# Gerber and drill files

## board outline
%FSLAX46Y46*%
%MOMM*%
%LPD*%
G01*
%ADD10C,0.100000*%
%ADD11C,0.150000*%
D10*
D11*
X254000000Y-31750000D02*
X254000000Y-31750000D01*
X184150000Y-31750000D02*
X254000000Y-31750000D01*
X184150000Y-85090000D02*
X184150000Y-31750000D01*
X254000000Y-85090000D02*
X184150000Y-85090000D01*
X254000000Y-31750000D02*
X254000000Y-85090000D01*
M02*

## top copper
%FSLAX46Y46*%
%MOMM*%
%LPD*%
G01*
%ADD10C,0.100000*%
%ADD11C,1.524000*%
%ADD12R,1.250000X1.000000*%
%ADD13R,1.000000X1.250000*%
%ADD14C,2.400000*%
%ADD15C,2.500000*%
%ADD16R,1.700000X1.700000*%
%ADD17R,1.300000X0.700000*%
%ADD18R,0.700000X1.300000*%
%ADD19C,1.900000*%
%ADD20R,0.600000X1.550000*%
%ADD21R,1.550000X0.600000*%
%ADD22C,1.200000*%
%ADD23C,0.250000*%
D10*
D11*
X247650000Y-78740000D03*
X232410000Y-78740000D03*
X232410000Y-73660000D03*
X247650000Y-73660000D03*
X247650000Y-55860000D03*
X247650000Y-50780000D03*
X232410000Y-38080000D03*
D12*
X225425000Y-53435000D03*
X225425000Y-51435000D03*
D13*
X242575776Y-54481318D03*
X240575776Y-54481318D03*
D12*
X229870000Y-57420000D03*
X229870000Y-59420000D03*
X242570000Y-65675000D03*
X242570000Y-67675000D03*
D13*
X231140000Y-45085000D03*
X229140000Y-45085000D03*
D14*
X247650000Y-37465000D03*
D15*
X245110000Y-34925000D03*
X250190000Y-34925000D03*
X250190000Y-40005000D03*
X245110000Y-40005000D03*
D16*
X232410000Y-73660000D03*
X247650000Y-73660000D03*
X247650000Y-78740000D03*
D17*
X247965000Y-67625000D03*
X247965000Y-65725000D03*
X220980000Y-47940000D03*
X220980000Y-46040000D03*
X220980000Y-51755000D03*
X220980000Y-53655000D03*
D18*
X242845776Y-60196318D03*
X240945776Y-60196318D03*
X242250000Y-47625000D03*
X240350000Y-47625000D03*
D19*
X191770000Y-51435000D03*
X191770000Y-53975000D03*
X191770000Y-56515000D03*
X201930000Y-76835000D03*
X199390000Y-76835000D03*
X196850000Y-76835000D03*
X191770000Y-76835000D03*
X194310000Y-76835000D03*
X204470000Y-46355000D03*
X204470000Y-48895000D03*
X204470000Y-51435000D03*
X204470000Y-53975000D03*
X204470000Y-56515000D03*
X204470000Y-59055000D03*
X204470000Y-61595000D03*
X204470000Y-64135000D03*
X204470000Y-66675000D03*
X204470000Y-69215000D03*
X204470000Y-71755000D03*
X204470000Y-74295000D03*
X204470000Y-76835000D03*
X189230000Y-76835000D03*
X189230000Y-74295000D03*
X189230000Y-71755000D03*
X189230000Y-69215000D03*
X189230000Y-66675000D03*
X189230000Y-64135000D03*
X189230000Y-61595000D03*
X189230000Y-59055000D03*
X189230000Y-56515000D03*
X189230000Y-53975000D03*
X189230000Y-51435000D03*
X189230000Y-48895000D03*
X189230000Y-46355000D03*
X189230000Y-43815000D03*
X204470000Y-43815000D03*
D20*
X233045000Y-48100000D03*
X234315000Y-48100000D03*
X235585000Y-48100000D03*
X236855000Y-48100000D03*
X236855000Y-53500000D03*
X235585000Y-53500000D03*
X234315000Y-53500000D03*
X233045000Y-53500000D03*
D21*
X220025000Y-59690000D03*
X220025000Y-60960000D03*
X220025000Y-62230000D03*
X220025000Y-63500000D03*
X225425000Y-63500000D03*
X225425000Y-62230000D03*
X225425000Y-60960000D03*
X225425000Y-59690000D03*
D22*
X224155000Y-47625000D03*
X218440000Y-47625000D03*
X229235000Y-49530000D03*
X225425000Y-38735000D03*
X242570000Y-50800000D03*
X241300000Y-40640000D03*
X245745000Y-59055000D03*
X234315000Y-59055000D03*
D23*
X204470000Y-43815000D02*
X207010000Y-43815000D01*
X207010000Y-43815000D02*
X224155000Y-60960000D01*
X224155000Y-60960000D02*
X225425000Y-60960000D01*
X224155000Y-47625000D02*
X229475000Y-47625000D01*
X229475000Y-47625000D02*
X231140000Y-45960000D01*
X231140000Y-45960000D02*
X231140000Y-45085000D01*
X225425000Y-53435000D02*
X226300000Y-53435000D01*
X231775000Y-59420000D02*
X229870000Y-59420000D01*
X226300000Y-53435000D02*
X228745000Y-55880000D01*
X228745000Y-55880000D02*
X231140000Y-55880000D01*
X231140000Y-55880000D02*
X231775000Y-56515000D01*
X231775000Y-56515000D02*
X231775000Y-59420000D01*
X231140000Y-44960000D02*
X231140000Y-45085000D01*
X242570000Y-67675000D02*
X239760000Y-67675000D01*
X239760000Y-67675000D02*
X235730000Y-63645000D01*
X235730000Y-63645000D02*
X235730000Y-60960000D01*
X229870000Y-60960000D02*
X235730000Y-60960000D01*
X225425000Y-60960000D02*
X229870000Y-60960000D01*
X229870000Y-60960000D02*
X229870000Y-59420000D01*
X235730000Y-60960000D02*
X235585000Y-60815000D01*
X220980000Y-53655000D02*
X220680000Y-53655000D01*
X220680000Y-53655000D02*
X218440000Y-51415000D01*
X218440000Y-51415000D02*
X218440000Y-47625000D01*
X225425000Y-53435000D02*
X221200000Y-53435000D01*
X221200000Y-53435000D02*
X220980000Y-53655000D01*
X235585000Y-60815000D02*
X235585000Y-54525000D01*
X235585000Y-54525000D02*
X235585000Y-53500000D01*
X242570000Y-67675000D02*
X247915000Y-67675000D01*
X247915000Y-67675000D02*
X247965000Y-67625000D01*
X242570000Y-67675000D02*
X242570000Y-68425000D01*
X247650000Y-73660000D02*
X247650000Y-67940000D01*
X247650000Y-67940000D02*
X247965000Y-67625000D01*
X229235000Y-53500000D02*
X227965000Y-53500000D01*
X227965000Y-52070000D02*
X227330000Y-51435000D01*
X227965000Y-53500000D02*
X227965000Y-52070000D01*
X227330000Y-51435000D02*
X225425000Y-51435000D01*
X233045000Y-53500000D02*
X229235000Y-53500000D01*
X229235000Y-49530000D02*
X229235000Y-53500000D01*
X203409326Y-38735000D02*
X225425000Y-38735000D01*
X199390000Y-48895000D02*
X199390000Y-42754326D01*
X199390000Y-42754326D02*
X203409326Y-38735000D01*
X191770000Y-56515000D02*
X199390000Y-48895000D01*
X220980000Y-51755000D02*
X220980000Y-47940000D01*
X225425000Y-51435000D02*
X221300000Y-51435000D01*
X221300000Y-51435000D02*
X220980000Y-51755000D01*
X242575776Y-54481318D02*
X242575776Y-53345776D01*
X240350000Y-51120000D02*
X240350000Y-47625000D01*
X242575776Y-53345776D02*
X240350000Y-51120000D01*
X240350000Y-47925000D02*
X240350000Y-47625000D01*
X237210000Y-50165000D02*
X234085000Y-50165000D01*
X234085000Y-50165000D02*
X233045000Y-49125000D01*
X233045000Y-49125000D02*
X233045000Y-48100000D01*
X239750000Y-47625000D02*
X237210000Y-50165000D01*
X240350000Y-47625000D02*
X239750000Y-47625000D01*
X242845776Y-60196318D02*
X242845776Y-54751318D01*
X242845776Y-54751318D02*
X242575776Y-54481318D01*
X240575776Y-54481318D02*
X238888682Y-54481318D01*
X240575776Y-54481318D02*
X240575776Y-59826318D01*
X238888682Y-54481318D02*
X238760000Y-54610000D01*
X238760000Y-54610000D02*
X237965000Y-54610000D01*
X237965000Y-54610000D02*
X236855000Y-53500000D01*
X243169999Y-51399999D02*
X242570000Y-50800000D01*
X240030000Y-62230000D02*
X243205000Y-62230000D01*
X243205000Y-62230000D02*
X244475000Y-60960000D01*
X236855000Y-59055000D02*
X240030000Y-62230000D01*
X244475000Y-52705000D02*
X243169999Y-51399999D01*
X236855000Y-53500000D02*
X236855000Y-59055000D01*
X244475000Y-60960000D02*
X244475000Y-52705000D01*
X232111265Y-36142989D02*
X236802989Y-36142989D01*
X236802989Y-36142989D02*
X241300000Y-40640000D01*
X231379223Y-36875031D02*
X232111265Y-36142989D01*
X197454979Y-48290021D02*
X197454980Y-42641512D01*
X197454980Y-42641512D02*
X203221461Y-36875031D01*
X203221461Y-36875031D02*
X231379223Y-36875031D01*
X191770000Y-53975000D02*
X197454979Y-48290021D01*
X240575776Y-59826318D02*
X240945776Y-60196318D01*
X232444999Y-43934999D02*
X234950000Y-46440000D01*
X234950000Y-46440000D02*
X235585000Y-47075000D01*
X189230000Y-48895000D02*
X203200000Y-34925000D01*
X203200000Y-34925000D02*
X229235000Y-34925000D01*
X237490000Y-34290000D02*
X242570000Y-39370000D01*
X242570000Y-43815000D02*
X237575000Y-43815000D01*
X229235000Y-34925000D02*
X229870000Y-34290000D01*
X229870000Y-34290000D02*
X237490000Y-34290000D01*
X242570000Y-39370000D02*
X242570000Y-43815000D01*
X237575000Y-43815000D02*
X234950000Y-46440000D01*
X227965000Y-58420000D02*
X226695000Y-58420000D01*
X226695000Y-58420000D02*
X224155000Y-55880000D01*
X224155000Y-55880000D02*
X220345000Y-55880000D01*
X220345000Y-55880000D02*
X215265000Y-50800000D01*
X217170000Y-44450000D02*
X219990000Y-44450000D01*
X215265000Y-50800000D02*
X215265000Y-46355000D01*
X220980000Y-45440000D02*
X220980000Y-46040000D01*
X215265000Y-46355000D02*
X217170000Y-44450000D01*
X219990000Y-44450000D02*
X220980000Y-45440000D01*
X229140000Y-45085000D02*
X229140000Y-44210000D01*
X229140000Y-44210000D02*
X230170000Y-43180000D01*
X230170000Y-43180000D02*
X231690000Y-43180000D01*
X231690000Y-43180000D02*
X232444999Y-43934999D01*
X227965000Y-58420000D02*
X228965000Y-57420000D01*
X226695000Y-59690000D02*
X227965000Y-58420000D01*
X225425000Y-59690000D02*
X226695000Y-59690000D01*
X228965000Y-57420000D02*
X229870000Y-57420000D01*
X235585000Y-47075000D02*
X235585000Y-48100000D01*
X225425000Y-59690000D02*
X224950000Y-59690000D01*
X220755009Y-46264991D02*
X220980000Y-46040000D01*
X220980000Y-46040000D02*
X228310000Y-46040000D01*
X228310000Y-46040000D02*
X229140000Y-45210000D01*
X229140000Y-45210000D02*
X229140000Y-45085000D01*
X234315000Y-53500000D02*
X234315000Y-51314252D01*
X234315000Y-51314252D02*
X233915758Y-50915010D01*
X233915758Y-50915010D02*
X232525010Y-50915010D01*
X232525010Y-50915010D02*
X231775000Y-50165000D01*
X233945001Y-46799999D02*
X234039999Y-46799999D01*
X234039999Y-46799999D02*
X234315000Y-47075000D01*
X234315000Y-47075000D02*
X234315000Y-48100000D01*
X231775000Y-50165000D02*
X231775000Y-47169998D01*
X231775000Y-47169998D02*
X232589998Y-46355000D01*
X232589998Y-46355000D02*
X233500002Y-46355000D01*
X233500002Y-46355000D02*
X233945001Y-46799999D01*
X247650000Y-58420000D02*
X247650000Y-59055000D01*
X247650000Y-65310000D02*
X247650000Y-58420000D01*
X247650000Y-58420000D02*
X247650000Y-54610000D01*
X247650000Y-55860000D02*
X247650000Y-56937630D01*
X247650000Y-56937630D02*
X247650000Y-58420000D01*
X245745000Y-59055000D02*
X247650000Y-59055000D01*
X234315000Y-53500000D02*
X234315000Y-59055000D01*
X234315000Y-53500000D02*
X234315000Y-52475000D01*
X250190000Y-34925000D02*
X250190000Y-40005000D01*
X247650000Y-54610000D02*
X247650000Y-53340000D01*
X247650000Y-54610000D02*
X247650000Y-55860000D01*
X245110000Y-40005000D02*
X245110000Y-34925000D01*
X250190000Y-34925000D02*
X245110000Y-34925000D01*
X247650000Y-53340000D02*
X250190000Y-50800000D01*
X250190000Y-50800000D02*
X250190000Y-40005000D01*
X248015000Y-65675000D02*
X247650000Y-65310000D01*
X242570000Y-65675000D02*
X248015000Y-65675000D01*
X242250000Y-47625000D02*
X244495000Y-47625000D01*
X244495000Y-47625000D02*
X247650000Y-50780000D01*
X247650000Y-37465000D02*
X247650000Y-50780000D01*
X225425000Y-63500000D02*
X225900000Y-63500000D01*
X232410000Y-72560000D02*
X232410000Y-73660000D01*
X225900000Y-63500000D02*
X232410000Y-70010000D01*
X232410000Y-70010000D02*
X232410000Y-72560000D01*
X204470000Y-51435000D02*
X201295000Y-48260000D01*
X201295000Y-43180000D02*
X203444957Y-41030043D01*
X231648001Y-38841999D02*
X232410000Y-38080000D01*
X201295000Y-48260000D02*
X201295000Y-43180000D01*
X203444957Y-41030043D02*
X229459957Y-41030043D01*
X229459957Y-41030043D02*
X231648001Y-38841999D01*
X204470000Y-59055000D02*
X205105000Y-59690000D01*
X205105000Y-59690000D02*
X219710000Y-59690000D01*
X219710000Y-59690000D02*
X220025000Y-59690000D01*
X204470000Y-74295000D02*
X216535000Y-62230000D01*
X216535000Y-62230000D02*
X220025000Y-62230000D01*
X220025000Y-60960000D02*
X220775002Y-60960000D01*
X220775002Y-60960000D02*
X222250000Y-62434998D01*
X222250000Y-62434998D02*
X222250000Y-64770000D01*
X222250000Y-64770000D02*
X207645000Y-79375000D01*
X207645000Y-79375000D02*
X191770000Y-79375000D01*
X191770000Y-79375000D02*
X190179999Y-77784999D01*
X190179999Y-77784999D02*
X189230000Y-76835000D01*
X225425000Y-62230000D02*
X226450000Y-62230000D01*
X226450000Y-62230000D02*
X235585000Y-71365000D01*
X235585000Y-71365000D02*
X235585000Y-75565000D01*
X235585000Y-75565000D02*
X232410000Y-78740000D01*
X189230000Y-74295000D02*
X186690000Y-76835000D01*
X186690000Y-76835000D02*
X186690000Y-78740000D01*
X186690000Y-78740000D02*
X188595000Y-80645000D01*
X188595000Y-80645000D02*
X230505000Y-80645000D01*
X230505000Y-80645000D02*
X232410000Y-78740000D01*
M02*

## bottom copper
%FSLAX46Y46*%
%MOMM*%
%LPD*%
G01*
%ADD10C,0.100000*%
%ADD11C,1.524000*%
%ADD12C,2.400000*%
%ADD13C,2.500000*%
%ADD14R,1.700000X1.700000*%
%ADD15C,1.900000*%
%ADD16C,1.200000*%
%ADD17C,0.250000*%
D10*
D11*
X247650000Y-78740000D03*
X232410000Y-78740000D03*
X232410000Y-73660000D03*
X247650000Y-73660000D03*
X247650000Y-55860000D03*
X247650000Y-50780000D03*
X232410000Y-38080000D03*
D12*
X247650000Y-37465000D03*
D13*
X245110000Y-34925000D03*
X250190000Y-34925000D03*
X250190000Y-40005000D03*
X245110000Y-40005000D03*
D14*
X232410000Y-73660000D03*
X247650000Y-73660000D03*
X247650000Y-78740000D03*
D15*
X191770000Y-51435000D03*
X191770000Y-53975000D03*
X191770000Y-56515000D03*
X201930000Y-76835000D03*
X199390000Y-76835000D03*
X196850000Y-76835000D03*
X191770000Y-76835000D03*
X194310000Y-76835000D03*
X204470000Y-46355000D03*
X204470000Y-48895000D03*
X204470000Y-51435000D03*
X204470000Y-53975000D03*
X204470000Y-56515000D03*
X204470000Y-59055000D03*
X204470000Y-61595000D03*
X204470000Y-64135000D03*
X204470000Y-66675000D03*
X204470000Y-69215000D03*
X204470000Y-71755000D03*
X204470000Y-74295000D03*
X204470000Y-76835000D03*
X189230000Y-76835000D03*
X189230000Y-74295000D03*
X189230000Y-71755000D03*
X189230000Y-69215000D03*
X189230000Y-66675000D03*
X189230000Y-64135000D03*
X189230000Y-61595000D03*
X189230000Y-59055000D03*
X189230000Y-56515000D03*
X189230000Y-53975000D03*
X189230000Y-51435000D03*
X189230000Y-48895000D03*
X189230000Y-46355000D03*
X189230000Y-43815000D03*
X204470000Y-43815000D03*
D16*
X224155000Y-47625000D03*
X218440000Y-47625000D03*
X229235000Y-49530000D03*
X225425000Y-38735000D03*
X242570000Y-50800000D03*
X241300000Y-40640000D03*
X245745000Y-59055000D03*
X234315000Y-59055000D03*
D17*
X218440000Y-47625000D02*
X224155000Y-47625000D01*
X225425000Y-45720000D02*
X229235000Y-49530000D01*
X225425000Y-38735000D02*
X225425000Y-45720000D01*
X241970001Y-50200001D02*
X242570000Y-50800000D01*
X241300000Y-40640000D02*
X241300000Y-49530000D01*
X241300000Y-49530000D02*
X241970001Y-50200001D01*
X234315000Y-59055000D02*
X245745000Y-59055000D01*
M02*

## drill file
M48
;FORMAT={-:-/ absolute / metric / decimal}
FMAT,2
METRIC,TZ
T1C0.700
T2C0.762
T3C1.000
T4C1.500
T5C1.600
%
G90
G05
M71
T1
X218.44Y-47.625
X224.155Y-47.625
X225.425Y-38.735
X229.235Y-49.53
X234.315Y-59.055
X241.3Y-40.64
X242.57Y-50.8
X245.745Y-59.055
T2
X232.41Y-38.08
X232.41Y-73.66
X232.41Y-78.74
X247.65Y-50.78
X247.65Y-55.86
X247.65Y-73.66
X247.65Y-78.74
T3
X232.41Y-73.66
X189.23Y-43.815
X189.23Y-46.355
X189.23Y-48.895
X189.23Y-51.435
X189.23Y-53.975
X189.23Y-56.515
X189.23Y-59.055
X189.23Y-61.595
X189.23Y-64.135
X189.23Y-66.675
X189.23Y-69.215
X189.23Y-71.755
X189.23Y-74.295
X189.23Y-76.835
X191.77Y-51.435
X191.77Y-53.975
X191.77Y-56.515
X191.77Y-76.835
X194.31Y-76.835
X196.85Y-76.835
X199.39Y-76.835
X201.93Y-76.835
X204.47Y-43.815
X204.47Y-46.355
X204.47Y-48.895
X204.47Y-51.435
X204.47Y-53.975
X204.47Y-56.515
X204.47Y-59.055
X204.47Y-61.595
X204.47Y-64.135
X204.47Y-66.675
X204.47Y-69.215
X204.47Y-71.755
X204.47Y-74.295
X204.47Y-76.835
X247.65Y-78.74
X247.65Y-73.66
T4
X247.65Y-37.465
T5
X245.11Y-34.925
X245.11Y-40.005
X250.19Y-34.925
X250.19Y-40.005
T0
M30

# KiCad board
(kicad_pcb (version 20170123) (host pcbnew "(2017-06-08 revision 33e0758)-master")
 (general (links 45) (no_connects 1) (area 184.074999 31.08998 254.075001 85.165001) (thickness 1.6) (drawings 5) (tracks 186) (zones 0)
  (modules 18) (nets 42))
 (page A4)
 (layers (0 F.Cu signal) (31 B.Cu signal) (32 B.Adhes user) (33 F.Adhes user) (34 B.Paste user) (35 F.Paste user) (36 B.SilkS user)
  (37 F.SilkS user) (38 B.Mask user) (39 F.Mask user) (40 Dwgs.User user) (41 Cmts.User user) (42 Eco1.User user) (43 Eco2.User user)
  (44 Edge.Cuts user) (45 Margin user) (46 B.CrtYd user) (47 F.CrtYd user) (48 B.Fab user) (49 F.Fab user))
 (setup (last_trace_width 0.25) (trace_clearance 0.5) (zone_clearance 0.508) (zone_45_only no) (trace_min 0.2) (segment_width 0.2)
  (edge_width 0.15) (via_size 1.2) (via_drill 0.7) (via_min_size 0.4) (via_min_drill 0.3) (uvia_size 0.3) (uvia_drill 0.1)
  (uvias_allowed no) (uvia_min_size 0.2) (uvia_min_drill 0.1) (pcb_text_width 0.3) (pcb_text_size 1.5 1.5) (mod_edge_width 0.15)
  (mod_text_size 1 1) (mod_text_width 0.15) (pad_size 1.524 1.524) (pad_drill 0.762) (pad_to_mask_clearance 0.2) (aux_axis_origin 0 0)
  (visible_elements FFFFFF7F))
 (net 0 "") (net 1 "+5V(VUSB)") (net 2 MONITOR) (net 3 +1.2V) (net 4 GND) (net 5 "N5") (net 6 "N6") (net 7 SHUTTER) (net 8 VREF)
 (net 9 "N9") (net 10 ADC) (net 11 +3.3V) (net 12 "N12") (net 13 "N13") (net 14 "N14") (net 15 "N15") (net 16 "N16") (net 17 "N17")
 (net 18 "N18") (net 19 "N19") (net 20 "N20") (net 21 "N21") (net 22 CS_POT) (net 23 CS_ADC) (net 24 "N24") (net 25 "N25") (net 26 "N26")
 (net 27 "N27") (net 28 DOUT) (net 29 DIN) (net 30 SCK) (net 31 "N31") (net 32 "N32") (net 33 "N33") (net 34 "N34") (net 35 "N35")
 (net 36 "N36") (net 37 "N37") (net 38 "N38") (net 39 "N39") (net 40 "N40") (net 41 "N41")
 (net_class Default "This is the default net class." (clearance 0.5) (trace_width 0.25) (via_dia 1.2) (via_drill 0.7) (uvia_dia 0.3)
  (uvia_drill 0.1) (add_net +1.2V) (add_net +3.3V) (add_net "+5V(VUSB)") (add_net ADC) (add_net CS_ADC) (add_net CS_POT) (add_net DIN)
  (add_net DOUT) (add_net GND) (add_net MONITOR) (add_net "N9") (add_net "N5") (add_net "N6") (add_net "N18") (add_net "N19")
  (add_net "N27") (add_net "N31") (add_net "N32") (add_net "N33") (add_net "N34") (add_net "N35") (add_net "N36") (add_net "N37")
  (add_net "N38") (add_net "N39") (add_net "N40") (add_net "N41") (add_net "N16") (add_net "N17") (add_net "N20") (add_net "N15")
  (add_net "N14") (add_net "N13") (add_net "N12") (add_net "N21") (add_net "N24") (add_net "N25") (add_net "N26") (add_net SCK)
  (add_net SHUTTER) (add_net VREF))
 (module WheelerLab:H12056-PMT (layer B.Cu) (at 232.41 38.08 270)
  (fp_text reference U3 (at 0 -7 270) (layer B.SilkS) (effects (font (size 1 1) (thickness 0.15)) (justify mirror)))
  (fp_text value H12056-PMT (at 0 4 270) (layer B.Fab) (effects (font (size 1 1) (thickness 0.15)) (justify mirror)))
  (pad 4 thru_hole circle (at 40.66 -15.24 270) (size 1.524 1.524) (drill 0.762) (layers *.Cu *.Mask) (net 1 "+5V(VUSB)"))
  (pad 3 thru_hole circle (at 40.66 0 270) (size 1.524 1.524) (drill 0.762) (layers *.Cu *.Mask) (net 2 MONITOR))
  (pad 2 thru_hole circle (at 35.58 0 270) (size 1.524 1.524) (drill 0.762) (layers *.Cu *.Mask) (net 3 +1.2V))
  (pad 5 thru_hole circle (at 35.58 -15.24 270) (size 1.524 1.524) (drill 0.762) (layers *.Cu *.Mask) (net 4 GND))
  (pad 6 thru_hole circle (at 17.78 -15.24 270) (size 1.524 1.524) (drill 0.762) (layers *.Cu *.Mask) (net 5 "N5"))
  (pad 7 thru_hole circle (at 12.7 -15.24 270) (size 1.524 1.524) (drill 0.762) (layers *.Cu *.Mask) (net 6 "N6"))
  (pad 1 thru_hole circle (at 0 0 270) (size 1.524 1.524) (drill 0.762) (layers *.Cu *.Mask) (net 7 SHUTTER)))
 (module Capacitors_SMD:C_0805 (layer F.Cu) (at 225.425 52.435 90)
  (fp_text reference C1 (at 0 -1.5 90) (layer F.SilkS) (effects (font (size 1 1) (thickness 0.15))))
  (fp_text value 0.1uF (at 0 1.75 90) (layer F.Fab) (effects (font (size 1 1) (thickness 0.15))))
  (pad 1 smd rect (at -1 0 90) (size 1 1.25) (layers F.Cu F.Paste F.Mask) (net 4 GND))
  (pad 2 smd rect (at 1 0 90) (size 1 1.25) (layers F.Cu F.Paste F.Mask) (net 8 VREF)))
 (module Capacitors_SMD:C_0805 (layer F.Cu) (at 241.575776 54.481318)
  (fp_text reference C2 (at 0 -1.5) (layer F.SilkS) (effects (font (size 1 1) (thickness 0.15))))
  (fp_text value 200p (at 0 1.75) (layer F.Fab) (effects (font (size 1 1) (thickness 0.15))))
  (pad 2 smd rect (at 1 0) (size 1 1.25) (layers F.Cu F.Paste F.Mask) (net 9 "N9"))
  (pad 1 smd rect (at -1 0) (size 1 1.25) (layers F.Cu F.Paste F.Mask) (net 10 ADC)))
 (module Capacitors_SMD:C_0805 (layer F.Cu) (at 229.87 58.42 90)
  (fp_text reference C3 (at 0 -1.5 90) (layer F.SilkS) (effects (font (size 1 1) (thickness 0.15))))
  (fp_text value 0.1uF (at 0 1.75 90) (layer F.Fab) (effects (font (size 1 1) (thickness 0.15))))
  (pad 2 smd rect (at 1 0 90) (size 1 1.25) (layers F.Cu F.Paste F.Mask) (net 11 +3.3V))
  (pad 1 smd rect (at -1 0 90) (size 1 1.25) (layers F.Cu F.Paste F.Mask) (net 4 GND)))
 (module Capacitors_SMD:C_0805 (layer F.Cu) (at 242.57 66.675 270)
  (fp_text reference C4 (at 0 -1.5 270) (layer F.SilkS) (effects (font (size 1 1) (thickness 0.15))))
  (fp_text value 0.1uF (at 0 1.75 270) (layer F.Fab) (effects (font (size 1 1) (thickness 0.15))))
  (pad 1 smd rect (at -1 0 270) (size 1 1.25) (layers F.Cu F.Paste F.Mask) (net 5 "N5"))
  (pad 2 smd rect (at 1 0 270) (size 1 1.25) (layers F.Cu F.Paste F.Mask) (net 4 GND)))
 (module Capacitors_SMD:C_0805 (layer F.Cu) (at 230.14 45.085)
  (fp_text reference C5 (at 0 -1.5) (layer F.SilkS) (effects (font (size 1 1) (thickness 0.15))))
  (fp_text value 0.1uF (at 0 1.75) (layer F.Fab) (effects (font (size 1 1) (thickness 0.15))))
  (pad 2 smd rect (at 1 0) (size 1 1.25) (layers F.Cu F.Paste F.Mask) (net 4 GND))
  (pad 1 smd rect (at -1 0) (size 1 1.25) (layers F.Cu F.Paste F.Mask) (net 11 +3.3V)))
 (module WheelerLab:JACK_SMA (layer F.Cu) (at 247.65 37.465)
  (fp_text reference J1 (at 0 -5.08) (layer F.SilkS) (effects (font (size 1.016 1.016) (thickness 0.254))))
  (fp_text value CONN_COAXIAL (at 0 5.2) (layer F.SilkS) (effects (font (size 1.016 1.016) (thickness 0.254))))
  (pad 1 thru_hole circle (at 0 0) (size 2.4 2.4) (drill 1.5) (layers *.Cu *.Mask F.SilkS) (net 6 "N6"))
  (pad 2 thru_hole circle (at -2.54 -2.54) (size 2.5 2.5) (drill 1.6) (layers *.Cu *.Mask F.SilkS) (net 5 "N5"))
  (pad 2 thru_hole circle (at 2.54 -2.54) (size 2.5 2.5) (drill 1.6) (layers *.Cu *.Mask F.SilkS) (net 5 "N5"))
  (pad 2 thru_hole circle (at 2.54 2.54) (size 2.5 2.5) (drill 1.6) (layers *.Cu *.Mask F.SilkS) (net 5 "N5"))
  (pad 2 thru_hole circle (at -2.54 2.54) (size 2.5 2.5) (drill 1.6) (layers *.Cu *.Mask F.SilkS) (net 5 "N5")))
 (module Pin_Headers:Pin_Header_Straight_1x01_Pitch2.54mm (layer F.Cu) (at 232.41 73.66)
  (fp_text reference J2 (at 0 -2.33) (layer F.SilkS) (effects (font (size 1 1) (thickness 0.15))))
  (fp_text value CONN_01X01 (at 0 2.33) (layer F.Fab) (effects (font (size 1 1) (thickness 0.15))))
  (pad 1 thru_hole rect (at 0 0) (size 1.7 1.7) (drill 1) (layers *.Cu *.Mask) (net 3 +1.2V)))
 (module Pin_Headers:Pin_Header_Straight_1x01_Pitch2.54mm (layer F.Cu) (at 247.65 73.66)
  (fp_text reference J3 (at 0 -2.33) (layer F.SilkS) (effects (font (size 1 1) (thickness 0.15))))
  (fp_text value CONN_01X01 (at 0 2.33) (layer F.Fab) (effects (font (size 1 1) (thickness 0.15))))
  (pad 1 thru_hole rect (at 0 0) (size 1.7 1.7) (drill 1) (layers *.Cu *.Mask) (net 4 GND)))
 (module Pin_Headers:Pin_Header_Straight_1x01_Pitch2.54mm (layer F.Cu) (at 247.65 78.74)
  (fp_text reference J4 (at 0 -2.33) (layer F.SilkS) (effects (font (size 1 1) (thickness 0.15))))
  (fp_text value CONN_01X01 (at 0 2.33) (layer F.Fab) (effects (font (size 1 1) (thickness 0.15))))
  (pad 1 thru_hole rect (at 0 0) (size 1.7 1.7) (drill 1) (layers *.Cu *.Mask) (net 1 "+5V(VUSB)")))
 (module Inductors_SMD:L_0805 (layer F.Cu) (at 247.965 66.675 270)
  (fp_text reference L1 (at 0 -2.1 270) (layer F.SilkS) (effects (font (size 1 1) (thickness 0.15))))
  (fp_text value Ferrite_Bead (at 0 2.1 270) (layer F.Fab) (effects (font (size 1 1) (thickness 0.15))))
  (pad 2 smd rect (at 0.95 0 270) (size 0.7 1.3) (layers F.Cu F.Paste F.Mask) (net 4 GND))
  (pad 1 smd rect (at -0.95 0 270) (size 0.7 1.3) (layers F.Cu F.Paste F.Mask) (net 5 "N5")))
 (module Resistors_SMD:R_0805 (layer F.Cu) (at 220.98 46.99 270)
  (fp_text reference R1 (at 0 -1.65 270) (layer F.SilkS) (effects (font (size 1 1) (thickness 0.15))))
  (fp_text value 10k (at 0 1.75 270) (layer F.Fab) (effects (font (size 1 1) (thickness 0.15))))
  (pad 2 smd rect (at 0.95 0 270) (size 0.7 1.3) (layers F.Cu F.Paste F.Mask) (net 8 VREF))
  (pad 1 smd rect (at -0.95 0 270) (size 0.7 1.3) (layers F.Cu F.Paste F.Mask) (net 11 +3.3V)))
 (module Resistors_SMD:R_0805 (layer F.Cu) (at 220.98 52.705 270)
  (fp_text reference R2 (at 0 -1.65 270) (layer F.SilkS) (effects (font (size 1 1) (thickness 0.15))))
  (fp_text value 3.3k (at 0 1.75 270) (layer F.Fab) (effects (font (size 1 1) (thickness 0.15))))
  (pad 1 smd rect (at -0.95 0 270) (size 0.7 1.3) (layers F.Cu F.Paste F.Mask) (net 8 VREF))
  (pad 2 smd rect (at 0.95 0 270) (size 0.7 1.3) (layers F.Cu F.Paste F.Mask) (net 4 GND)))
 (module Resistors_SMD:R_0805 (layer F.Cu) (at 241.895776 60.196318)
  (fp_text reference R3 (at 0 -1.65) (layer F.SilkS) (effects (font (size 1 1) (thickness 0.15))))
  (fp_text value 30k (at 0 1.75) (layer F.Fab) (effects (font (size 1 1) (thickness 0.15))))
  (pad 2 smd rect (at 0.95 0) (size 0.7 1.3) (layers F.Cu F.Paste F.Mask) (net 9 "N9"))
  (pad 1 smd rect (at -0.95 0) (size 0.7 1.3) (layers F.Cu F.Paste F.Mask) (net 10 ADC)))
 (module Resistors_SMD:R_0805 (layer F.Cu) (at 241.3 47.625 180)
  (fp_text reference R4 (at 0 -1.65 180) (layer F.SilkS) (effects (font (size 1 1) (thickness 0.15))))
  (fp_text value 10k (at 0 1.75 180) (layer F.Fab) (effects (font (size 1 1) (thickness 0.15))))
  (pad 1 smd rect (at -0.95 0 180) (size 0.7 1.3) (layers F.Cu F.Paste F.Mask) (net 6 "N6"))
  (pad 2 smd rect (at 0.95 0 180) (size 0.7 1.3) (layers F.Cu F.Paste F.Mask) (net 9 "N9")))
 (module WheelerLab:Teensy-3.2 (layer B.Cu) (at 196.85 60.071 270)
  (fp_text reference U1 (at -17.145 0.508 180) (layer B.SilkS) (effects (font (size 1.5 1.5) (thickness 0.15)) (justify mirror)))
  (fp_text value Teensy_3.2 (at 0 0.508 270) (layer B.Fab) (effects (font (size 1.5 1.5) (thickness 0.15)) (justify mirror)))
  (pad 35 thru_hole circle (at -8.636 5.08 270) (size 1.9 1.9) (drill 1) (layers *.Cu *.Mask B.SilkS) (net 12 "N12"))
  (pad 34 thru_hole circle (at -6.096 5.08 270) (size 1.9 1.9) (drill 1) (layers *.Cu *.Mask B.SilkS) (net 10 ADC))
  (pad 33 thru_hole circle (at -3.556 5.08 270) (size 1.9 1.9) (drill 1) (layers *.Cu *.Mask B.SilkS) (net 8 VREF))
  (pad 32 thru_hole circle (at 16.764 -5.08 270) (size 1.9 1.9) (drill 1) (layers *.Cu *.Mask B.SilkS) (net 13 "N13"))
  (pad 31 thru_hole circle (at 16.764 -2.54 270) (size 1.9 1.9) (drill 1) (layers *.Cu *.Mask B.SilkS) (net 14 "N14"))
  (pad 30 thru_hole circle (at 16.764 0 270) (size 1.9 1.9) (drill 1) (layers *.Cu *.Mask B.SilkS) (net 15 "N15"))
  (pad 28 thru_hole circle (at 16.764 5.08 270) (size 1.9 1.9) (drill 1) (layers *.Cu *.Mask B.SilkS) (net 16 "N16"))
  (pad 29 thru_hole circle (at 16.764 2.54 270) (size 1.9 1.9) (drill 1) (layers *.Cu *.Mask B.SilkS) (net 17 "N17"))
  (pad 0 thru_hole circle (at -13.716 -7.62 270) (size 1.9 1.9) (drill 1) (layers *.Cu *.Mask B.SilkS) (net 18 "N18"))
  (pad 1 thru_hole circle (at -11.176 -7.62 270) (size 1.9 1.9) (drill 1) (layers *.Cu *.Mask B.SilkS) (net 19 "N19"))
  (pad 2 thru_hole circle (at -8.636 -7.62 270) (size 1.9 1.9) (drill 1) (layers *.Cu *.Mask B.SilkS) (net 7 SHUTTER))
  (pad 3 thru_hole circle (at -6.096 -7.62 270) (size 1.9 1.9) (drill 1) (layers *.Cu *.Mask B.SilkS) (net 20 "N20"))
  (pad 4 thru_hole circle (at -3.556 -7.62 270) (size 1.9 1.9) (drill 1) (layers *.Cu *.Mask B.SilkS) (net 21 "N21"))
  (pad 5 thru_hole circle (at -1.016 -7.62 270) (size 1.9 1.9) (drill 1) (layers *.Cu *.Mask B.SilkS) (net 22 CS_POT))
  (pad 6 thru_hole circle (at 1.524 -7.62 270) (size 1.9 1.9) (drill 1) (layers *.Cu *.Mask B.SilkS) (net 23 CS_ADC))
  (pad 7 thru_hole circle (at 4.064 -7.62 270) (size 1.9 1.9) (drill 1) (layers *.Cu *.Mask B.SilkS) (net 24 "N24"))
  (pad 8 thru_hole circle (at 6.604 -7.62 270) (size 1.9 1.9) (drill 1) (layers *.Cu *.Mask B.SilkS) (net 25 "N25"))
  (pad 9 thru_hole circle (at 9.144 -7.62 270) (size 1.9 1.9) (drill 1) (layers *.Cu *.Mask B.SilkS) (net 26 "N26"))
  (pad 10 thru_hole circle (at 11.684 -7.62 270) (size 1.9 1.9) (drill 1) (layers *.Cu *.Mask B.SilkS) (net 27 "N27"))
  (pad 11 thru_hole circle (at 14.224 -7.62 270) (size 1.9 1.9) (drill 1) (layers *.Cu *.Mask B.SilkS) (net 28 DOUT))
  (pad 12 thru_hole circle (at 16.764 -7.62 270) (size 1.9 1.9) (drill 1) (layers *.Cu *.Mask B.SilkS) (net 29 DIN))
  (pad 13 thru_hole circle (at 16.764 7.62 270) (size 1.9 1.9) (drill 1) (layers *.Cu *.Mask B.SilkS) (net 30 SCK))
  (pad 14 thru_hole circle (at 14.224 7.62 270) (size 1.9 1.9) (drill 1) (layers *.Cu *.Mask B.SilkS) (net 2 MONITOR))
  (pad 15 thru_hole circle (at 11.684 7.62 270) (size 1.9 1.9) (drill 1) (layers *.Cu *.Mask B.SilkS) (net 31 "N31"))
  (pad 16 thru_hole circle (at 9.144 7.62 270) (size 1.9 1.9) (drill 1) (layers *.Cu *.Mask B.SilkS) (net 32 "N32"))
  (pad 17 thru_hole circle (at 6.604 7.62 270) (size 1.9 1.9) (drill 1) (layers *.Cu *.Mask B.SilkS) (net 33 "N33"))
  (pad 18 thru_hole circle (at 4.064 7.62 270) (size 1.9 1.9) (drill 1) (layers *.Cu *.Mask B.SilkS) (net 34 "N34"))
  (pad 19 thru_hole circle (at 1.524 7.62 270) (size 1.9 1.9) (drill 1) (layers *.Cu *.Mask B.SilkS) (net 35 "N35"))
  (pad 20 thru_hole circle (at -1.016 7.62 270) (size 1.9 1.9) (drill 1) (layers *.Cu *.Mask B.SilkS) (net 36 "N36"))
  (pad 21 thru_hole circle (at -3.556 7.62 270) (size 1.9 1.9) (drill 1) (layers *.Cu *.Mask B.SilkS) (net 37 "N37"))
  (pad 22 thru_hole circle (at -6.096 7.62 270) (size 1.9 1.9) (drill 1) (layers *.Cu *.Mask B.SilkS) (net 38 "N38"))
  (pad 23 thru_hole circle (at -8.636 7.62 270) (size 1.9 1.9) (drill 1) (layers *.Cu *.Mask B.SilkS) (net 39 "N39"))
  (pad 24 thru_hole circle (at -11.176 7.62 270) (size 1.9 1.9) (drill 1) (layers *.Cu *.Mask B.SilkS) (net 11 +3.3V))
  (pad 25 thru_hole circle (at -13.716 7.62 270) (size 1.9 1.9) (drill 1) (layers *.Cu *.Mask B.SilkS) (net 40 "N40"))
  (pad 26 thru_hole circle (at -16.256 7.62 270) (size 1.9 1.9) (drill 1) (layers *.Cu *.Mask B.SilkS) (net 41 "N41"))
  (pad 27 thru_hole circle (at -16.256 -7.62 270) (size 1.9 1.9) (drill 1) (layers *.Cu *.Mask B.SilkS) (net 4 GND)))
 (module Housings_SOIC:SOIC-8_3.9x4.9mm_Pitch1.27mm (layer F.Cu) (at 234.95 50.8 90)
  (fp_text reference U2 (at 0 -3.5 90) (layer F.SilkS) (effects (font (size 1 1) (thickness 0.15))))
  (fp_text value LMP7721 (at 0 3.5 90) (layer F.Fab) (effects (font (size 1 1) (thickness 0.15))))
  (pad 8 smd rect (at 2.7 -1.905 90) (size 1.55 0.6) (layers F.Cu F.Paste F.Mask) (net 9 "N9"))
  (pad 7 smd rect (at 2.7 -0.635 90) (size 1.55 0.6) (layers F.Cu F.Paste F.Mask) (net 5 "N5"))
  (pad 6 smd rect (at 2.7 0.635 90) (size 1.55 0.6) (layers F.Cu F.Paste F.Mask) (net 11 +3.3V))
  (pad 5 smd rect (at 2.7 1.905 90) (size 1.55 0.6) (layers F.Cu F.Paste F.Mask))
  (pad 4 smd rect (at -2.7 1.905 90) (size 1.55 0.6) (layers F.Cu F.Paste F.Mask) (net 10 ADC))
  (pad 3 smd rect (at -2.7 0.635 90) (size 1.55 0.6) (layers F.Cu F.Paste F.Mask) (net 4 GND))
  (pad 2 smd rect (at -2.7 -0.635 90) (size 1.55 0.6) (layers F.Cu F.Paste F.Mask) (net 5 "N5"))
  (pad 1 smd rect (at -2.7 -1.905 90) (size 1.55 0.6) (layers F.Cu F.Paste F.Mask) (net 8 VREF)))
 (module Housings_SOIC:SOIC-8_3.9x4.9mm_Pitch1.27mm (layer F.Cu) (at 222.725 61.595)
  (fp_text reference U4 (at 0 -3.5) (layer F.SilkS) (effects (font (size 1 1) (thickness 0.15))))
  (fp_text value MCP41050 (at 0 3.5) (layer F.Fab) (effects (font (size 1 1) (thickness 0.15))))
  (pad 1 smd rect (at -2.7 -1.905) (size 1.55 0.6) (layers F.Cu F.Paste F.Mask) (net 22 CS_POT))
  (pad 2 smd rect (at -2.7 -0.635) (size 1.55 0.6) (layers F.Cu F.Paste F.Mask) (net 30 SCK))
  (pad 3 smd rect (at -2.7 0.635) (size 1.55 0.6) (layers F.Cu F.Paste F.Mask) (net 28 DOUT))
  (pad 4 smd rect (at -2.7 1.905) (size 1.55 0.6) (layers F.Cu F.Paste F.Mask) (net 4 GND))
  (pad 5 smd rect (at 2.7 1.905) (size 1.55 0.6) (layers F.Cu F.Paste F.Mask) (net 3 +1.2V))
  (pad 6 smd rect (at 2.7 0.635) (size 1.55 0.6) (layers F.Cu F.Paste F.Mask) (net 2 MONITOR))
  (pad 7 smd rect (at 2.7 -0.635) (size 1.55 0.6) (layers F.Cu F.Paste F.Mask) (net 4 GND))
  (pad 8 smd rect (at 2.7 -1.905) (size 1.55 0.6) (layers F.Cu F.Paste F.Mask) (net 11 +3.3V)))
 (gr_line (start 254 31.75) (end 254 31.75) (layer Edge.Cuts) (width 0.15))
 (gr_line (start 184.15 31.75) (end 254 31.75) (layer Edge.Cuts) (width 0.15))
 (gr_line (start 184.15 85.09) (end 184.15 31.75) (layer Edge.Cuts) (width 0.15))
 (gr_line (start 254 85.09) (end 184.15 85.09) (layer Edge.Cuts) (width 0.15))
 (gr_line (start 254 31.75) (end 254 85.09) (layer Edge.Cuts) (width 0.15))
 (segment (start 204.47 43.815) (end 207.01 43.815) (width 0.25) (layer F.Cu) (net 4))
 (segment (start 207.01 43.815) (end 224.155 60.96) (width 0.25) (layer F.Cu) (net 4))
 (segment (start 224.155 60.96) (end 225.425 60.96) (width 0.25) (layer F.Cu) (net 4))
 (segment (start 224.155 47.625) (end 229.475 47.625) (width 0.25) (layer F.Cu) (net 4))
 (segment (start 229.475 47.625) (end 231.14 45.96) (width 0.25) (layer F.Cu) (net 4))
 (segment (start 231.14 45.96) (end 231.14 45.085) (width 0.25) (layer F.Cu) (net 4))
 (segment (start 218.44 47.625) (end 224.155 47.625) (width 0.25) (layer B.Cu) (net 4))
 (via (at 224.155 47.625) (size 1.2) (drill 0.7) (layers F.Cu B.Cu) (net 4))
 (via (at 218.44 47.625) (size 1.2) (drill 0.7) (layers F.Cu B.Cu) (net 4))
 (segment (start 225.425 53.435) (end 226.3 53.435) (width 0.25) (layer F.Cu) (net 4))
 (segment (start 231.775 59.42) (end 229.87 59.42) (width 0.25) (layer F.Cu) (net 4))
 (segment (start 226.3 53.435) (end 228.745 55.88) (width 0.25) (layer F.Cu) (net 4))
 (segment (start 228.745 55.88) (end 231.14 55.88) (width 0.25) (layer F.Cu) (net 4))
 (segment (start 231.14 55.88) (end 231.775 56.515) (width 0.25) (layer F.Cu) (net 4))
 (segment (start 231.775 56.515) (end 231.775 59.42) (width 0.25) (layer F.Cu) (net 4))
 (segment (start 231.14 44.96) (end 231.14 45.085) (width 0.25) (layer F.Cu) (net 4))
 (segment (start 242.57 67.675) (end 239.76 67.675) (width 0.25) (layer F.Cu) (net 4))
 (segment (start 239.76 67.675) (end 235.73 63.645) (width 0.25) (layer F.Cu) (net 4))
 (segment (start 235.73 63.645) (end 235.73 60.96) (width 0.25) (layer F.Cu) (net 4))
 (segment (start 229.87 60.96) (end 235.73 60.96) (width 0.25) (layer F.Cu) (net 4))
 (segment (start 225.425 60.96) (end 229.87 60.96) (width 0.25) (layer F.Cu) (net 4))
 (segment (start 229.87 60.96) (end 229.87 59.42) (width 0.25) (layer F.Cu) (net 4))
 (segment (start 235.73 60.96) (end 235.585 60.815) (width 0.25) (layer F.Cu) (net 4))
 (segment (start 220.98 53.655) (end 220.68 53.655) (width 0.25) (layer F.Cu) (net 4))
 (segment (start 220.68 53.655) (end 218.44 51.415) (width 0.25) (layer F.Cu) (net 4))
 (segment (start 218.44 51.415) (end 218.44 47.625) (width 0.25) (layer F.Cu) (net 4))
 (segment (start 225.425 53.435) (end 221.2 53.435) (width 0.25) (layer F.Cu) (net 4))
 (segment (start 221.2 53.435) (end 220.98 53.655) (width 0.25) (layer F.Cu) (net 4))
 (segment (start 235.585 60.815) (end 235.585 54.525) (width 0.25) (layer F.Cu) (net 4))
 (segment (start 235.585 54.525) (end 235.585 53.5) (width 0.25) (layer F.Cu) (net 4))
 (segment (start 242.57 67.675) (end 247.915 67.675) (width 0.25) (layer F.Cu) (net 4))
 (segment (start 247.915 67.675) (end 247.965 67.625) (width 0.25) (layer F.Cu) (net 4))
 (segment (start 242.57 67.675) (end 242.57 68.425) (width 0.25) (layer F.Cu) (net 4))
 (segment (start 247.65 73.66) (end 247.65 67.94) (width 0.25) (layer F.Cu) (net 4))
 (segment (start 247.65 67.94) (end 247.965 67.625) (width 0.25) (layer F.Cu) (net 4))
 (segment (start 229.235 53.5) (end 227.965 53.5) (width 0.25) (layer F.Cu) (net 8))
 (segment (start 227.965 52.07) (end 227.33 51.435) (width 0.25) (layer F.Cu) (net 8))
 (segment (start 227.965 53.5) (end 227.965 52.07) (width 0.25) (layer F.Cu) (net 8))
 (segment (start 227.33 51.435) (end 225.425 51.435) (width 0.25) (layer F.Cu) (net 8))
 (segment (start 233.045 53.5) (end 229.235 53.5) (width 0.25) (layer F.Cu) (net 8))
 (segment (start 229.235 49.53) (end 229.235 53.5) (width 0.25) (layer F.Cu) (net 8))
 (segment (start 225.425 45.72) (end 229.235 49.53) (width 0.25) (layer B.Cu) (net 8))
 (via (at 229.235 49.53) (size 1.2) (drill 0.7) (layers F.Cu B.Cu) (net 8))
 (segment (start 225.425 38.735) (end 225.425 45.72) (width 0.25) (layer B.Cu) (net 8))
 (via (at 225.425 38.735) (size 1.2) (drill 0.7) (layers F.Cu B.Cu) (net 8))
 (segment (start 203.409326 38.735) (end 225.425 38.735) (width 0.25) (layer F.Cu) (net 8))
 (segment (start 199.39 48.895) (end 199.39 42.754326) (width 0.25) (layer F.Cu) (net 8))
 (segment (start 199.39 42.754326) (end 203.409326 38.735) (width 0.25) (layer F.Cu) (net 8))
 (segment (start 191.77 56.515) (end 199.39 48.895) (width 0.25) (layer F.Cu) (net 8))
 (segment (start 220.98 51.755) (end 220.98 47.94) (width 0.25) (layer F.Cu) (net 8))
 (segment (start 225.425 51.435) (end 221.3 51.435) (width 0.25) (layer F.Cu) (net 8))
 (segment (start 221.3 51.435) (end 220.98 51.755) (width 0.25) (layer F.Cu) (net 8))
 (segment (start 242.575776 54.481318) (end 242.575776 53.345776) (width 0.25) (layer F.Cu) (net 9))
 (segment (start 240.35 51.12) (end 240.35 47.625) (width 0.25) (layer F.Cu) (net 9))
 (segment (start 242.575776 53.345776) (end 240.35 51.12) (width 0.25) (layer F.Cu) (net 9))
 (segment (start 240.35 47.925) (end 240.35 47.625) (width 0.25) (layer F.Cu) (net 9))
 (segment (start 237.21 50.165) (end 234.085 50.165) (width 0.25) (layer F.Cu) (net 9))
 (segment (start 234.085 50.165) (end 233.045 49.125) (width 0.25) (layer F.Cu) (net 9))
 (segment (start 233.045 49.125) (end 233.045 48.1) (width 0.25) (layer F.Cu) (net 9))
 (segment (start 239.75 47.625) (end 237.21 50.165) (width 0.25) (layer F.Cu) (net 9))
 (segment (start 240.35 47.625) (end 239.75 47.625) (width 0.25) (layer F.Cu) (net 9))
 (segment (start 242.845776 60.196318) (end 242.845776 54.751318) (width 0.25) (layer F.Cu) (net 9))
 (segment (start 242.845776 54.751318) (end 242.575776 54.481318) (width 0.25) (layer F.Cu) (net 9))
 (segment (start 240.575776 54.481318) (end 238.888682 54.481318) (width 0.25) (layer F.Cu) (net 10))
 (segment (start 240.575776 54.481318) (end 240.575776 59.826318) (width 0.25) (layer F.Cu) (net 10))
 (segment (start 238.888682 54.481318) (end 238.76 54.61) (width 0.25) (layer F.Cu) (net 10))
 (segment (start 238.76 54.61) (end 237.965 54.61) (width 0.25) (layer F.Cu) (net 10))
 (segment (start 237.965 54.61) (end 236.855 53.5) (width 0.25) (layer F.Cu) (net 10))
 (segment (start 241.970001 50.200001) (end 242.57 50.8) (width 0.25) (layer B.Cu) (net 10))
 (segment (start 241.3 40.64) (end 241.3 49.53) (width 0.25) (layer B.Cu) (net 10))
 (segment (start 243.169999 51.399999) (end 242.57 50.8) (width 0.25) (layer F.Cu) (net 10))
 (segment (start 240.03 62.23) (end 243.205 62.23) (width 0.25) (layer F.Cu) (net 10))
 (segment (start 243.205 62.23) (end 244.475 60.96) (width 0.25) (layer F.Cu) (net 10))
 (segment (start 236.855 59.055) (end 240.03 62.23) (width 0.25) (layer F.Cu) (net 10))
 (segment (start 241.3 49.53) (end 241.970001 50.200001) (width 0.25) (layer B.Cu) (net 10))
 (segment (start 244.475 52.705) (end 243.169999 51.399999) (width 0.25) (layer F.Cu) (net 10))
 (segment (start 236.855 53.5) (end 236.855 59.055) (width 0.25) (layer F.Cu) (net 10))
 (via (at 242.57 50.8) (size 1.2) (drill 0.7) (layers F.Cu B.Cu) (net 10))
 (segment (start 244.475 60.96) (end 244.475 52.705) (width 0.25) (layer F.Cu) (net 10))
 (via (at 241.3 40.64) (size 1.2) (drill 0.7) (layers F.Cu B.Cu) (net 10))
 (segment (start 232.111265 36.142989) (end 236.802989 36.142989) (width 0.25) (layer F.Cu) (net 10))
 (segment (start 236.802989 36.142989) (end 241.3 40.64) (width 0.25) (layer F.Cu) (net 10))
 (segment (start 231.379223 36.875031) (end 232.111265 36.142989) (width 0.25) (layer F.Cu) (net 10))
 (segment (start 197.454979 48.290021) (end 197.45498 42.641512) (width 0.25) (layer F.Cu) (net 10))
 (segment (start 197.45498 42.641512) (end 203.221461 36.875031) (width 0.25) (layer F.Cu) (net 10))
 (segment (start 203.221461 36.875031) (end 231.379223 36.875031) (width 0.25) (layer F.Cu) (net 10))
 (segment (start 191.77 53.975) (end 197.454979 48.290021) (width 0.25) (layer F.Cu) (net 10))
 (segment (start 240.575776 59.826318) (end 240.945776 60.196318) (width 0.25) (layer F.Cu) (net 10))
 (segment (start 232.444999 43.934999) (end 234.95 46.44) (width 0.25) (layer F.Cu) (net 11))
 (segment (start 234.95 46.44) (end 235.585 47.075) (width 0.25) (layer F.Cu) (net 11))
 (segment (start 189.23 48.895) (end 203.2 34.925) (width 0.25) (layer F.Cu) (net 11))
 (segment (start 203.2 34.925) (end 229.235 34.925) (width 0.25) (layer F.Cu) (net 11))
 (segment (start 237.49 34.29) (end 242.57 39.37) (width 0.25) (layer F.Cu) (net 11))
 (segment (start 242.57 43.815) (end 237.575 43.815) (width 0.25) (layer F.Cu) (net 11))
 (segment (start 229.235 34.925) (end 229.87 34.29) (width 0.25) (layer F.Cu) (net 11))
 (segment (start 229.87 34.29) (end 237.49 34.29) (width 0.25) (layer F.Cu) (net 11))
 (segment (start 242.57 39.37) (end 242.57 43.815) (width 0.25) (layer F.Cu) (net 11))
 (segment (start 237.575 43.815) (end 234.95 46.44) (width 0.25) (layer F.Cu) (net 11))
 (segment (start 227.965 58.42) (end 226.695 58.42) (width 0.25) (layer F.Cu) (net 11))
 (segment (start 226.695 58.42) (end 224.155 55.88) (width 0.25) (layer F.Cu) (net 11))
 (segment (start 224.155 55.88) (end 220.345 55.88) (width 0.25) (layer F.Cu) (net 11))
 (segment (start 220.345 55.88) (end 215.265 50.8) (width 0.25) (layer F.Cu) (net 11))
 (segment (start 217.17 44.45) (end 219.99 44.45) (width 0.25) (layer F.Cu) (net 11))
 (segment (start 215.265 50.8) (end 215.265 46.355) (width 0.25) (layer F.Cu) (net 11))
 (segment (start 220.98 45.44) (end 220.98 46.04) (width 0.25) (layer F.Cu) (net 11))
 (segment (start 215.265 46.355) (end 217.17 44.45) (width 0.25) (layer F.Cu) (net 11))
 (segment (start 219.99 44.45) (end 220.98 45.44) (width 0.25) (layer F.Cu) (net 11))
 (segment (start 229.14 45.085) (end 229.14 44.21) (width 0.25) (layer F.Cu) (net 11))
 (segment (start 229.14 44.21) (end 230.17 43.18) (width 0.25) (layer F.Cu) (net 11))
 (segment (start 230.17 43.18) (end 231.69 43.18) (width 0.25) (layer F.Cu) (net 11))
 (segment (start 231.69 43.18) (end 232.444999 43.934999) (width 0.25) (layer F.Cu) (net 11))
 (segment (start 227.965 58.42) (end 228.965 57.42) (width 0.25) (layer F.Cu) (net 11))
 (segment (start 226.695 59.69) (end 227.965 58.42) (width 0.25) (layer F.Cu) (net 11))
 (segment (start 225.425 59.69) (end 226.695 59.69) (width 0.25) (layer F.Cu) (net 11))
 (segment (start 228.965 57.42) (end 229.87 57.42) (width 0.25) (layer F.Cu) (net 11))
 (segment (start 235.585 47.075) (end 235.585 48.1) (width 0.25) (layer F.Cu) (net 11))
 (segment (start 225.425 59.69) (end 224.95 59.69) (width 0.25) (layer F.Cu) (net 11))
 (segment (start 220.755009 46.264991) (end 220.98 46.04) (width 0.25) (layer F.Cu) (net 11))
 (segment (start 220.98 46.04) (end 228.31 46.04) (width 0.25) (layer F.Cu) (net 11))
 (segment (start 228.31 46.04) (end 229.14 45.21) (width 0.25) (layer F.Cu) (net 11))
 (segment (start 229.14 45.21) (end 229.14 45.085) (width 0.25) (layer F.Cu) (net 11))
 (segment (start 234.315 53.5) (end 234.315 51.314252) (width 0.25) (layer F.Cu) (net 5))
 (segment (start 234.315 51.314252) (end 233.915758 50.91501) (width 0.25) (layer F.Cu) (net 5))
 (segment (start 233.915758 50.91501) (end 232.52501 50.91501) (width 0.25) (layer F.Cu) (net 5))
 (segment (start 232.52501 50.91501) (end 231.775 50.165) (width 0.25) (layer F.Cu) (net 5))
 (segment (start 233.945001 46.799999) (end 234.039999 46.799999) (width 0.25) (layer F.Cu) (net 5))
 (segment (start 234.039999 46.799999) (end 234.315 47.075) (width 0.25) (layer F.Cu) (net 5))
 (segment (start 234.315 47.075) (end 234.315 48.1) (width 0.25) (layer F.Cu) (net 5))
 (segment (start 231.775 50.165) (end 231.775 47.169998) (width 0.25) (layer F.Cu) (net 5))
 (segment (start 231.775 47.169998) (end 232.589998 46.355) (width 0.25) (layer F.Cu) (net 5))
 (segment (start 232.589998 46.355) (end 233.500002 46.355) (width 0.25) (layer F.Cu) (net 5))
 (segment (start 233.500002 46.355) (end 233.945001 46.799999) (width 0.25) (layer F.Cu) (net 5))
 (segment (start 247.65 58.42) (end 247.65 59.055) (width 0.25) (layer F.Cu) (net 5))
 (segment (start 247.65 65.31) (end 247.65 58.42) (width 0.25) (layer F.Cu) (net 5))
 (segment (start 247.65 58.42) (end 247.65 54.61) (width 0.25) (layer F.Cu) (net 5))
 (segment (start 247.65 55.86) (end 247.65 56.93763) (width 0.25) (layer F.Cu) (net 5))
 (segment (start 247.65 56.93763) (end 247.65 58.42) (width 0.25) (layer F.Cu) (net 5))
 (segment (start 245.745 59.055) (end 247.65 59.055) (width 0.25) (layer F.Cu) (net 5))
 (segment (start 234.315 59.055) (end 245.745 59.055) (width 0.25) (layer B.Cu) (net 5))
 (via (at 245.745 59.055) (size 1.2) (drill 0.7) (layers F.Cu B.Cu) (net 5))
 (segment (start 234.315 53.5) (end 234.315 59.055) (width 0.25) (layer F.Cu) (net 5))
 (via (at 234.315 59.055) (size 1.2) (drill 0.7) (layers F.Cu B.Cu) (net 5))
 (segment (start 234.315 53.5) (end 234.315 52.475) (width 0.25) (layer F.Cu) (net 5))
 (segment (start 250.19 34.925) (end 250.19 40.005) (width 0.25) (layer F.Cu) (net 5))
 (segment (start 247.65 54.61) (end 247.65 53.34) (width 0.25) (layer F.Cu) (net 5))
 (segment (start 247.65 54.61) (end 247.65 55.86) (width 0.25) (layer F.Cu) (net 5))
 (segment (start 245.11 40.005) (end 245.11 34.925) (width 0.25) (layer F.Cu) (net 5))
 (segment (start 250.19 34.925) (end 245.11 34.925) (width 0.25) (layer F.Cu) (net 5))
 (segment (start 247.65 53.34) (end 250.19 50.8) (width 0.25) (layer F.Cu) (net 5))
 (segment (start 250.19 50.8) (end 250.19 40.005) (width 0.25) (layer F.Cu) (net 5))
 (segment (start 248.015 65.675) (end 247.65 65.31) (width 0.25) (layer F.Cu) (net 5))
 (segment (start 242.57 65.675) (end 248.015 65.675) (width 0.25) (layer F.Cu) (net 5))
 (segment (start 242.25 47.625) (end 244.495 47.625) (width 0.25) (layer F.Cu) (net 6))
 (segment (start 244.495 47.625) (end 247.65 50.78) (width 0.25) (layer F.Cu) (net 6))
 (segment (start 247.65 37.465) (end 247.65 50.78) (width 0.25) (layer F.Cu) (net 6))
 (segment (start 225.425 63.5) (end 225.9 63.5) (width 0.25) (layer F.Cu) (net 3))
 (segment (start 232.41 72.56) (end 232.41 73.66) (width 0.25) (layer F.Cu) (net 3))
 (segment (start 225.9 63.5) (end 232.41 70.01) (width 0.25) (layer F.Cu) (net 3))
 (segment (start 232.41 70.01) (end 232.41 72.56) (width 0.25) (layer F.Cu) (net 3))
 (segment (start 204.47 51.435) (end 201.295 48.26) (width 0.25) (layer F.Cu) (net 7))
 (segment (start 201.295 43.18) (end 203.444957 41.030043) (width 0.25) (layer F.Cu) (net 7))
 (segment (start 231.648001 38.841999) (end 232.41 38.08) (width 0.25) (layer F.Cu) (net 7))
 (segment (start 201.295 48.26) (end 201.295 43.18) (width 0.25) (layer F.Cu) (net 7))
 (segment (start 203.444957 41.030043) (end 229.459957 41.030043) (width 0.25) (layer F.Cu) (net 7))
 (segment (start 229.459957 41.030043) (end 231.648001 38.841999) (width 0.25) (layer F.Cu) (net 7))
 (segment (start 204.47 59.055) (end 205.105 59.69) (width 0.25) (layer F.Cu) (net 22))
 (segment (start 205.105 59.69) (end 219.71 59.69) (width 0.25) (layer F.Cu) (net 22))
 (segment (start 219.71 59.69) (end 220.025 59.69) (width 0.25) (layer F.Cu) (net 22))
 (segment (start 204.47 74.295) (end 216.535 62.23) (width 0.25) (layer F.Cu) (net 28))
 (segment (start 216.535 62.23) (end 220.025 62.23) (width 0.25) (layer F.Cu) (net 28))
 (segment (start 220.025 60.96) (end 220.775002 60.96) (width 0.25) (layer F.Cu) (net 30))
 (segment (start 220.775002 60.96) (end 222.25 62.434998) (width 0.25) (layer F.Cu) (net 30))
 (segment (start 222.25 62.434998) (end 222.25 64.77) (width 0.25) (layer F.Cu) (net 30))
 (segment (start 222.25 64.77) (end 207.645 79.375) (width 0.25) (layer F.Cu) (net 30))
 (segment (start 207.645 79.375) (end 191.77 79.375) (width 0.25) (layer F.Cu) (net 30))
 (segment (start 191.77 79.375) (end 190.179999 77.784999) (width 0.25) (layer F.Cu) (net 30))
 (segment (start 190.179999 77.784999) (end 189.23 76.835) (width 0.25) (layer F.Cu) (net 30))
 (segment (start 225.425 62.23) (end 226.45 62.23) (width 0.25) (layer F.Cu) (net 2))
 (segment (start 226.45 62.23) (end 235.585 71.365) (width 0.25) (layer F.Cu) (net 2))
 (segment (start 235.585 71.365) (end 235.585 75.565) (width 0.25) (layer F.Cu) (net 2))
 (segment (start 235.585 75.565) (end 232.41 78.74) (width 0.25) (layer F.Cu) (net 2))
 (segment (start 189.23 74.295) (end 186.69 76.835) (width 0.25) (layer F.Cu) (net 2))
 (segment (start 186.69 76.835) (end 186.69 78.74) (width 0.25) (layer F.Cu) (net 2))
 (segment (start 186.69 78.74) (end 188.595 80.645) (width 0.25) (layer F.Cu) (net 2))
 (segment (start 188.595 80.645) (end 230.505 80.645) (width 0.25) (layer F.Cu) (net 2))
 (segment (start 230.505 80.645) (end 232.41 78.74) (width 0.25) (layer F.Cu) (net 2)))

